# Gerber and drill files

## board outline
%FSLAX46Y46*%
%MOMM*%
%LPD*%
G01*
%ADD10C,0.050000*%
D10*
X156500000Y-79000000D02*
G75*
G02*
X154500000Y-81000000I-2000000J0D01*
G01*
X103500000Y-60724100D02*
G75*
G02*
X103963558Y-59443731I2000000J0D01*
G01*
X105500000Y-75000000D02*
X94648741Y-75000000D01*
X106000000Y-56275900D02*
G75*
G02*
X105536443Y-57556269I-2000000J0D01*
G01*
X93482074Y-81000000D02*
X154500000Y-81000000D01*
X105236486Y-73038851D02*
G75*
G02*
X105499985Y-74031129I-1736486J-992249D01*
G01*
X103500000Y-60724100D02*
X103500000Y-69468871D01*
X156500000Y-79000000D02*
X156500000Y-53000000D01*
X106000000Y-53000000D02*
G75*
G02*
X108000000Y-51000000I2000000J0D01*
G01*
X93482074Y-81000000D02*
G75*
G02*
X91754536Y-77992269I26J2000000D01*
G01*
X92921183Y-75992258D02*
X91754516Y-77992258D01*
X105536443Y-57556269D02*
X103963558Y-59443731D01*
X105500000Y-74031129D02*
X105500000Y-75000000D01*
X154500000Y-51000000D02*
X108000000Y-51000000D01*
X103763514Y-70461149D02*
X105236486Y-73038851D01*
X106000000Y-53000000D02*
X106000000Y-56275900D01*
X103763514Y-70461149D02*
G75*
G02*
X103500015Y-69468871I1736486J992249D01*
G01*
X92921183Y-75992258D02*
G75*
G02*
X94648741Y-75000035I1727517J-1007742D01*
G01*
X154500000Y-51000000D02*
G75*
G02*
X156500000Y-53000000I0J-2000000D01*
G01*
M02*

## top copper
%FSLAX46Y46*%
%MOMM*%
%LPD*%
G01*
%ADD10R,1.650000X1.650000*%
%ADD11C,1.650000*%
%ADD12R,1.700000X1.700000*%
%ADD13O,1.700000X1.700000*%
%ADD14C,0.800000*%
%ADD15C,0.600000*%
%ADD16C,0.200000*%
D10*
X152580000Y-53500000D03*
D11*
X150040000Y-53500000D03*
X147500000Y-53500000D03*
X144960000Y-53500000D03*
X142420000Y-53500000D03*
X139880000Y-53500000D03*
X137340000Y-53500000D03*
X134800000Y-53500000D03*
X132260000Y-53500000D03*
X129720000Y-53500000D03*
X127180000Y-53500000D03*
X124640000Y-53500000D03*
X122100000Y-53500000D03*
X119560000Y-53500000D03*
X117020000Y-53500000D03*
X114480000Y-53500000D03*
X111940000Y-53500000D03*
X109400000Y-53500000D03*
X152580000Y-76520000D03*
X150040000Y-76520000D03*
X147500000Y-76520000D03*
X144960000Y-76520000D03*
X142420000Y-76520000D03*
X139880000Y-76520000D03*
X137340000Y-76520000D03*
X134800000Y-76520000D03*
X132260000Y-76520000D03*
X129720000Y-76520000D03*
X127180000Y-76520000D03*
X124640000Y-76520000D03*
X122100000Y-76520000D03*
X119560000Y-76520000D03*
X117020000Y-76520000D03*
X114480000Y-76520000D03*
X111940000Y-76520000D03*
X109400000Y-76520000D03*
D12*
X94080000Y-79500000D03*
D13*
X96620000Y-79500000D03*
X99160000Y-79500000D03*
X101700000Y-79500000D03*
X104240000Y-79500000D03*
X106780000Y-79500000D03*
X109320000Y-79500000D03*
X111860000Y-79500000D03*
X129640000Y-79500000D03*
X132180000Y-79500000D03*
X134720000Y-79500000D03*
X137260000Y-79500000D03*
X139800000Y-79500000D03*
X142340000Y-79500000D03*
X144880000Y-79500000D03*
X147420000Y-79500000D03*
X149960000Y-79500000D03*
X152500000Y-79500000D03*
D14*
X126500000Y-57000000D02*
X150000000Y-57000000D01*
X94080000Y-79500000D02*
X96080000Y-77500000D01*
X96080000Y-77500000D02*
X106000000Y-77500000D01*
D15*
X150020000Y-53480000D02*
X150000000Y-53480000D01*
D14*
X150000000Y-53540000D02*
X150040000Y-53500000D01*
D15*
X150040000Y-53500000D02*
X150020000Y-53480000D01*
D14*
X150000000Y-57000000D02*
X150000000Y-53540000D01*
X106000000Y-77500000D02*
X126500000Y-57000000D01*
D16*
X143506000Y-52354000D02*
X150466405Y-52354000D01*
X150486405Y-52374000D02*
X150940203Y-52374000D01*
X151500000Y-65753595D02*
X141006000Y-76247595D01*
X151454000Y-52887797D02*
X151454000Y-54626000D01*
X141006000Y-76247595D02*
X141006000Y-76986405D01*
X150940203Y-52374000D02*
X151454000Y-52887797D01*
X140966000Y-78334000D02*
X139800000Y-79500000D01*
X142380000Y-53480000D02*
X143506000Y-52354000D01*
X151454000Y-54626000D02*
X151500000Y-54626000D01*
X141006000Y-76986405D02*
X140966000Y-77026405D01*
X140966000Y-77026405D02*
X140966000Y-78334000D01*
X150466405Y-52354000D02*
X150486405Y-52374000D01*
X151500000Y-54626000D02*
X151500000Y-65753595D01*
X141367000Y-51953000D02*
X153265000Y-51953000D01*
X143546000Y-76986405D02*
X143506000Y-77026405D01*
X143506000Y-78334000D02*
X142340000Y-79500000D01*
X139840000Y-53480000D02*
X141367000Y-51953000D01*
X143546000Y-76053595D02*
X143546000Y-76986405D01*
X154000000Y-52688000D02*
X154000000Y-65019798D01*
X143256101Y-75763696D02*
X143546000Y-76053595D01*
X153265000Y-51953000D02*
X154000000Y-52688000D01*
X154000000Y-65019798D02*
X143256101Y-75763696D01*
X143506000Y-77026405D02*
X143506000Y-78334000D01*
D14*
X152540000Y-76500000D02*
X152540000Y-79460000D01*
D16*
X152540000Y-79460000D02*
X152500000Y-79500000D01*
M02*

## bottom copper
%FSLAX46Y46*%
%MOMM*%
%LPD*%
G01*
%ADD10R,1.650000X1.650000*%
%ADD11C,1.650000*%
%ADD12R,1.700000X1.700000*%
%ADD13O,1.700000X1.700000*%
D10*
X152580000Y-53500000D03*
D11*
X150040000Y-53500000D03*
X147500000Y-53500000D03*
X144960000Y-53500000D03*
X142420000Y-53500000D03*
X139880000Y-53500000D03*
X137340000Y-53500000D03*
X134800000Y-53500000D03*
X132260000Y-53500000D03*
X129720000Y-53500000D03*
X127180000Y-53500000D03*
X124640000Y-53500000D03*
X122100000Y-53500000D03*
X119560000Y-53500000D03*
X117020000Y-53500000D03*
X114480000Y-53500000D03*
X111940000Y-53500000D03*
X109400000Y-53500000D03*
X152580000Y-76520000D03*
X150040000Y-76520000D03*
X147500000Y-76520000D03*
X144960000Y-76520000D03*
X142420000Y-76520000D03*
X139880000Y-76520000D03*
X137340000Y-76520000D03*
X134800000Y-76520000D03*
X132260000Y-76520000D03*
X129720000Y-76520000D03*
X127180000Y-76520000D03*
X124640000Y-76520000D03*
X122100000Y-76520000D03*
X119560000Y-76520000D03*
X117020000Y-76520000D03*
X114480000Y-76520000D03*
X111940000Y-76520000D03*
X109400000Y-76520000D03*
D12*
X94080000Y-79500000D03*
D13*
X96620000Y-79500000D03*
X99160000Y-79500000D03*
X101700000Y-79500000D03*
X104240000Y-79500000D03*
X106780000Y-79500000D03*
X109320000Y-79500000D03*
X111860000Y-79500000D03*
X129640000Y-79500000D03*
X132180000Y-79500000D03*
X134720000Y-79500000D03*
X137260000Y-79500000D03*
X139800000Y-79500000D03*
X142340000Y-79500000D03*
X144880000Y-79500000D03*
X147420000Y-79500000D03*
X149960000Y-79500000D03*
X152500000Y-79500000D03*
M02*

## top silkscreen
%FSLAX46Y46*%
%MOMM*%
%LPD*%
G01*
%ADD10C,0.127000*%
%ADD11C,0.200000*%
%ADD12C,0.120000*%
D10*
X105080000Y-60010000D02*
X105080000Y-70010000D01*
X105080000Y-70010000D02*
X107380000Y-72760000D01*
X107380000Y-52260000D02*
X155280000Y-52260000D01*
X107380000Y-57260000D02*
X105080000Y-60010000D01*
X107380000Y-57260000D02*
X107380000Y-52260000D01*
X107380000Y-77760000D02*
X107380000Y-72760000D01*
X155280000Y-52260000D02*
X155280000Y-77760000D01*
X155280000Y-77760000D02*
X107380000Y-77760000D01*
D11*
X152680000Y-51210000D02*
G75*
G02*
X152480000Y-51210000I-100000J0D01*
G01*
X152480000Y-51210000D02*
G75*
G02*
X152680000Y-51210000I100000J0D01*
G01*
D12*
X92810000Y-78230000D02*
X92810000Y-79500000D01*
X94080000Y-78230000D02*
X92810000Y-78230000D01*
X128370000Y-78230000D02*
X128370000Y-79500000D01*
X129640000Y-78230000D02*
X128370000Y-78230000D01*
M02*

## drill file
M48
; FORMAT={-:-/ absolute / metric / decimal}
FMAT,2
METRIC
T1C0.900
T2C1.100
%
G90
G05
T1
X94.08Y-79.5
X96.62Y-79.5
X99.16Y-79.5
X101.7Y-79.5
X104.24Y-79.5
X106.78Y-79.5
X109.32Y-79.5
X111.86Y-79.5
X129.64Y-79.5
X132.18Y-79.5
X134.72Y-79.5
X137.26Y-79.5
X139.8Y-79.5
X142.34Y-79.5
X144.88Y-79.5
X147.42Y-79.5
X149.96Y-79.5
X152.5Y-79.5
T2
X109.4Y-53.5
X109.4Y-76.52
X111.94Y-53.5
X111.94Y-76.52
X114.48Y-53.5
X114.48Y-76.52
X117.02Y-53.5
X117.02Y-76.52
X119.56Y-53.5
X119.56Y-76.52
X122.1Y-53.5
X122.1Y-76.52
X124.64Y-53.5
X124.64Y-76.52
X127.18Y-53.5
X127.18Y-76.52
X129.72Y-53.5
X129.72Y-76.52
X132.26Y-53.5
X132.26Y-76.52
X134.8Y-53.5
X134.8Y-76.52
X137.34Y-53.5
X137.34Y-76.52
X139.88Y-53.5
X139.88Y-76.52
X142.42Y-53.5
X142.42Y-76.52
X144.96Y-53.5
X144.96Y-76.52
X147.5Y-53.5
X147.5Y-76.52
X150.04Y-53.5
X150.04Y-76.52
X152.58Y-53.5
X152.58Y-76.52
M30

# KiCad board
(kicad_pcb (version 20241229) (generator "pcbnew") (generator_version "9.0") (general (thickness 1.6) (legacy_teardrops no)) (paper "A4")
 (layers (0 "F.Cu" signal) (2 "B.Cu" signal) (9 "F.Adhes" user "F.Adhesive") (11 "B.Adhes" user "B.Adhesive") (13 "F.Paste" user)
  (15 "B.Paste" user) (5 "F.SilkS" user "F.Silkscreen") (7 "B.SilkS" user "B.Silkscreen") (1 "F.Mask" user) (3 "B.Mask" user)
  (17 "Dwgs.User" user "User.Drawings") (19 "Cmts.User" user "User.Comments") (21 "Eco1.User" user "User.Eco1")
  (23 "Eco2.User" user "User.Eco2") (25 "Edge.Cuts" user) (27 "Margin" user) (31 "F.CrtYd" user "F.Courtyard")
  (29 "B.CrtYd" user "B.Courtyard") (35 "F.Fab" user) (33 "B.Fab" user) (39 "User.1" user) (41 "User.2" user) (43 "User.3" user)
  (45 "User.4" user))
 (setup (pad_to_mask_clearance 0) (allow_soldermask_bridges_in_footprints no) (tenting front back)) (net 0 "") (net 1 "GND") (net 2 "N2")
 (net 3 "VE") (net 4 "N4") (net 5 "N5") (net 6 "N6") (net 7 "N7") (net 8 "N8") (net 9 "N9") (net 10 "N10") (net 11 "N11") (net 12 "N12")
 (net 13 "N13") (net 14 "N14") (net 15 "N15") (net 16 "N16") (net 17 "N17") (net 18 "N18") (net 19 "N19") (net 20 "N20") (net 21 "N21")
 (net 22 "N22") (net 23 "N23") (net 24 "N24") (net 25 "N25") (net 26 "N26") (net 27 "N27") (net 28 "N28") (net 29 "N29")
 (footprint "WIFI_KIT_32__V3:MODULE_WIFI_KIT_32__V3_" (layer "F.Cu") (at 130.18 65.01 -90)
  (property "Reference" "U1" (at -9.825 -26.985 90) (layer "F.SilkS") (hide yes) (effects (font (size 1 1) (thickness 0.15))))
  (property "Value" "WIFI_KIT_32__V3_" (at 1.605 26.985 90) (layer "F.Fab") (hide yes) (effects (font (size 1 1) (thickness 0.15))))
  (fp_line (start -5 25.1) (end 5 25.1) (stroke (width 0.127) (type solid)) (layer "F.SilkS"))
  (fp_line (start 5 25.1) (end 7.75 22.8) (stroke (width 0.127) (type solid)) (layer "F.SilkS"))
  (fp_line (start -12.75 22.8) (end -12.75 -25.1) (stroke (width 0.127) (type solid)) (layer "F.SilkS"))
  (fp_line (start -7.75 22.8) (end -5 25.1) (stroke (width 0.127) (type solid)) (layer "F.SilkS"))
  (fp_line (start -7.75 22.8) (end -12.75 22.8) (stroke (width 0.127) (type solid)) (layer "F.SilkS"))
  (fp_line (start 12.75 22.8) (end 7.75 22.8) (stroke (width 0.127) (type solid)) (layer "F.SilkS"))
  (fp_line (start -12.75 -25.1) (end 12.75 -25.1) (stroke (width 0.127) (type solid)) (layer "F.SilkS"))
  (fp_line (start 12.75 -25.1) (end 12.75 22.8) (stroke (width 0.127) (type solid)) (layer "F.SilkS"))
  (fp_circle (center -13.8 -22.4) (end -13.7 -22.4) (stroke (width 0.2) (type solid)) (fill no) (layer "F.SilkS"))
  (pad "J2_1" thru_hole rect (at -11.51 -22.4 270) (size 1.65 1.65) (drill 1.1) (layers "*.Cu" "*.Mask") (remove_unused_layers no)
   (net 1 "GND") (solder_mask_margin 0.102))
  (pad "J2_2" thru_hole circle (at -11.51 -19.86 270) (size 1.65 1.65) (drill 1.1) (layers "*.Cu" "*.Mask") (remove_unused_layers no)
   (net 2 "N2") (solder_mask_margin 0.102))
  (pad "J2_3" thru_hole circle (at -11.51 -17.32 270) (size 1.65 1.65) (drill 1.1) (layers "*.Cu" "*.Mask") (remove_unused_layers no)
   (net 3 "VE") (solder_mask_margin 0.102))
  (pad "J2_4" thru_hole circle (at -11.51 -14.78 270) (size 1.65 1.65) (drill 1.1) (layers "*.Cu" "*.Mask") (remove_unused_layers no)
   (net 3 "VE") (solder_mask_margin 0.102))
  (pad "J2_5" thru_hole circle (at -11.51 -12.24 270) (size 1.65 1.65) (drill 1.1) (layers "*.Cu" "*.Mask") (remove_unused_layers no)
   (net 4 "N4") (solder_mask_margin 0.102))
  (pad "J2_6" thru_hole circle (at -11.51 -9.7 270) (size 1.65 1.65) (drill 1.1) (layers "*.Cu" "*.Mask") (remove_unused_layers no)
   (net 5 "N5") (solder_mask_margin 0.102))
  (pad "J2_7" thru_hole circle (at -11.51 -7.16 270) (size 1.65 1.65) (drill 1.1) (layers "*.Cu" "*.Mask") (remove_unused_layers no)
   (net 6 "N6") (solder_mask_margin 0.102))
  (pad "J2_8" thru_hole circle (at -11.51 -4.62 270) (size 1.65 1.65) (drill 1.1) (layers "*.Cu" "*.Mask") (remove_unused_layers no)
   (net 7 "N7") (solder_mask_margin 0.102))
  (pad "J2_9" thru_hole circle (at -11.51 -2.08 270) (size 1.65 1.65) (drill 1.1) (layers "*.Cu" "*.Mask") (remove_unused_layers no)
   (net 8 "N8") (solder_mask_margin 0.102))
  (pad "J2_10" thru_hole circle (at -11.51 0.46 270) (size 1.65 1.65) (drill 1.1) (layers "*.Cu" "*.Mask") (remove_unused_layers no)
   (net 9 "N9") (solder_mask_margin 0.102))
  (pad "J2_11" thru_hole circle (at -11.51 3 270) (size 1.65 1.65) (drill 1.1) (layers "*.Cu" "*.Mask") (remove_unused_layers no)
   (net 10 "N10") (solder_mask_margin 0.102))
  (pad "J2_12" thru_hole circle (at -11.51 5.54 270) (size 1.65 1.65) (drill 1.1) (layers "*.Cu" "*.Mask") (remove_unused_layers no)
   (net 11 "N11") (solder_mask_margin 0.102))
  (pad "J2_13" thru_hole circle (at -11.51 8.08 270) (size 1.65 1.65) (drill 1.1) (layers "*.Cu" "*.Mask") (remove_unused_layers no)
   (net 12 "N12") (solder_mask_margin 0.102))
  (pad "J2_14" thru_hole circle (at -11.51 10.62 270) (size 1.65 1.65) (drill 1.1) (layers "*.Cu" "*.Mask") (remove_unused_layers no)
   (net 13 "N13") (solder_mask_margin 0.102))
  (pad "J2_15" thru_hole circle (at -11.51 13.16 270) (size 1.65 1.65) (drill 1.1) (layers "*.Cu" "*.Mask") (remove_unused_layers no)
   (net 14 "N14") (solder_mask_margin 0.102))
  (pad "J2_16" thru_hole circle (at -11.51 15.7 270) (size 1.65 1.65) (drill 1.1) (layers "*.Cu" "*.Mask") (remove_unused_layers no)
   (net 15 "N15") (solder_mask_margin 0.102))
  (pad "J2_17" thru_hole circle (at -11.51 18.24 270) (size 1.65 1.65) (drill 1.1) (layers "*.Cu" "*.Mask") (remove_unused_layers no)
   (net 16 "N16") (solder_mask_margin 0.102))
  (pad "J2_18" thru_hole circle (at -11.51 20.78 270) (size 1.65 1.65) (drill 1.1) (layers "*.Cu" "*.Mask") (remove_unused_layers no)
   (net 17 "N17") (solder_mask_margin 0.102))
  (pad "J3_1" thru_hole circle (at 11.51 -22.4 270) (size 1.65 1.65) (drill 1.1) (layers "*.Cu" "*.Mask") (remove_unused_layers no)
   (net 1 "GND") (solder_mask_margin 0.102))
  (pad "J3_2" thru_hole circle (at 11.51 -19.86 270) (size 1.65 1.65) (drill 1.1) (layers "*.Cu" "*.Mask") (remove_unused_layers no)
   (solder_mask_margin 0.102))
  (pad "J3_3" thru_hole circle (at 11.51 -17.32 270) (size 1.65 1.65) (drill 1.1) (layers "*.Cu" "*.Mask") (remove_unused_layers no)
   (solder_mask_margin 0.102))
  (pad "J3_4" thru_hole circle (at 11.51 -14.78 270) (size 1.65 1.65) (drill 1.1) (layers "*.Cu" "*.Mask") (remove_unused_layers no)
   (solder_mask_margin 0.102))
  (pad "J3_5" thru_hole circle (at 11.51 -12.24 270) (size 1.65 1.65) (drill 1.1) (layers "*.Cu" "*.Mask") (remove_unused_layers no)
   (solder_mask_margin 0.102))
  (pad "J3_6" thru_hole circle (at 11.51 -9.7 270) (size 1.65 1.65) (drill 1.1) (layers "*.Cu" "*.Mask") (remove_unused_layers no)
   (solder_mask_margin 0.102))
  (pad "J3_7" thru_hole circle (at 11.51 -7.16 270) (size 1.65 1.65) (drill 1.1) (layers "*.Cu" "*.Mask") (remove_unused_layers no)
   (solder_mask_margin 0.102))
  (pad "J3_8" thru_hole circle (at 11.51 -4.62 270) (size 1.65 1.65) (drill 1.1) (layers "*.Cu" "*.Mask") (remove_unused_layers no)
   (solder_mask_margin 0.102))
  (pad "J3_9" thru_hole circle (at 11.51 -2.08 270) (size 1.65 1.65) (drill 1.1) (layers "*.Cu" "*.Mask") (remove_unused_layers no)
   (solder_mask_margin 0.102))
  (pad "J3_10" thru_hole circle (at 11.51 0.46 270) (size 1.65 1.65) (drill 1.1) (layers "*.Cu" "*.Mask") (remove_unused_layers no)
   (solder_mask_margin 0.102))
  (pad "J3_11" thru_hole circle (at 11.51 3 270) (size 1.65 1.65) (drill 1.1) (layers "*.Cu" "*.Mask") (remove_unused_layers no)
   (solder_mask_margin 0.102))
  (pad "J3_12" thru_hole circle (at 11.51 5.54 270) (size 1.65 1.65) (drill 1.1) (layers "*.Cu" "*.Mask") (remove_unused_layers no)
   (solder_mask_margin 0.102))
  (pad "J3_13" thru_hole circle (at 11.51 8.08 270) (size 1.65 1.65) (drill 1.1) (layers "*.Cu" "*.Mask") (remove_unused_layers no)
   (solder_mask_margin 0.102))
  (pad "J3_14" thru_hole circle (at 11.51 10.62 270) (size 1.65 1.65) (drill 1.1) (layers "*.Cu" "*.Mask") (remove_unused_layers no)
   (solder_mask_margin 0.102))
  (pad "J3_15" thru_hole circle (at 11.51 13.16 270) (size 1.65 1.65) (drill 1.1) (layers "*.Cu" "*.Mask") (remove_unused_layers no)
   (solder_mask_margin 0.102))
  (pad "J3_16" thru_hole circle (at 11.51 15.7 270) (size 1.65 1.65) (drill 1.1) (layers "*.Cu" "*.Mask") (remove_unused_layers no)
   (solder_mask_margin 0.102))
  (pad "J3_17" thru_hole circle (at 11.51 18.24 270) (size 1.65 1.65) (drill 1.1) (layers "*.Cu" "*.Mask") (remove_unused_layers no)
   (solder_mask_margin 0.102))
  (pad "J3_18" thru_hole circle (at 11.51 20.78 270) (size 1.65 1.65) (drill 1.1) (layers "*.Cu" "*.Mask") (remove_unused_layers no)
   (solder_mask_margin 0.102)))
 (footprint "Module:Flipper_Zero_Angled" (layer "F.Cu") (at 94.08 79.5)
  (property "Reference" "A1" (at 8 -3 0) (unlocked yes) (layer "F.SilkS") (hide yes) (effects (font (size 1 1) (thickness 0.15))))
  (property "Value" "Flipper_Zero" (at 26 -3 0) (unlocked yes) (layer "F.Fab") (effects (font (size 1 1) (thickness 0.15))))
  (fp_line (start -1.27 -1.27) (end -1.27 0) (stroke (width 0.12) (type solid)) (layer "F.SilkS"))
  (fp_line (start 0 -1.27) (end -1.27 -1.27) (stroke (width 0.12) (type solid)) (layer "F.SilkS"))
  (fp_line (start 34.29 -1.27) (end 34.29 0) (stroke (width 0.12) (type solid)) (layer "F.SilkS"))
  (fp_line (start 35.56 -1.27) (end 34.29 -1.27) (stroke (width 0.12) (type solid)) (layer "F.SilkS"))
  (pad "1" thru_hole rect (at 0 0 90) (size 1.7 1.7) (drill 0.9) (layers "*.Cu" "*.Mask") (remove_unused_layers no) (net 2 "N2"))
  (pad "2" thru_hole oval (at 2.54 0 90) (size 1.7 1.7) (drill 0.9) (layers "*.Cu" "*.Mask") (remove_unused_layers no) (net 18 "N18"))
  (pad "3" thru_hole oval (at 5.08 0 90) (size 1.7 1.7) (drill 0.9) (layers "*.Cu" "*.Mask") (remove_unused_layers no) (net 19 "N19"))
  (pad "4" thru_hole oval (at 7.62 0 90) (size 1.7 1.7) (drill 0.9) (layers "*.Cu" "*.Mask") (remove_unused_layers no) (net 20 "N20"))
  (pad "5" thru_hole oval (at 10.16 0 90) (size 1.7 1.7) (drill 0.9) (layers "*.Cu" "*.Mask") (remove_unused_layers no) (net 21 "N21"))
  (pad "6" thru_hole oval (at 12.7 0 90) (size 1.7 1.7) (drill 0.9) (layers "*.Cu" "*.Mask") (remove_unused_layers no) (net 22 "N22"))
  (pad "7" thru_hole oval (at 15.24 0 90) (size 1.7 1.7) (drill 0.9) (layers "*.Cu" "*.Mask") (remove_unused_layers no) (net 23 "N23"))
  (pad "8" thru_hole oval (at 17.78 0 90) (size 1.7 1.7) (drill 0.9) (layers "*.Cu" "*.Mask") (remove_unused_layers no) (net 1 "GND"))
  (pad "9" thru_hole oval (at 35.56 0 90) (size 1.7 1.7) (drill 0.9) (layers "*.Cu" "*.Mask") (remove_unused_layers no) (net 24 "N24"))
  (pad "10" thru_hole oval (at 38.1 0 90) (size 1.7 1.7) (drill 0.9) (layers "*.Cu" "*.Mask") (remove_unused_layers no) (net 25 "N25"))
  (pad "11" thru_hole oval (at 40.64 0 90) (size 1.7 1.7) (drill 0.9) (layers "*.Cu" "*.Mask") (remove_unused_layers no) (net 1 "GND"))
  (pad "12" thru_hole oval (at 43.18 0 90) (size 1.7 1.7) (drill 0.9) (layers "*.Cu" "*.Mask") (remove_unused_layers no) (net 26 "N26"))
  (pad "13" thru_hole oval (at 45.72 0 90) (size 1.7 1.7) (drill 0.9) (layers "*.Cu" "*.Mask") (remove_unused_layers no) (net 4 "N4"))
  (pad "14" thru_hole oval (at 48.26 0 90) (size 1.7 1.7) (drill 0.9) (layers "*.Cu" "*.Mask") (remove_unused_layers no) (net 5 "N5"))
  (pad "15" thru_hole oval (at 50.8 0 90) (size 1.7 1.7) (drill 0.9) (layers "*.Cu" "*.Mask") (remove_unused_layers no) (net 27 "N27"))
  (pad "16" thru_hole oval (at 53.34 0 90) (size 1.7 1.7) (drill 0.9) (layers "*.Cu" "*.Mask") (remove_unused_layers no) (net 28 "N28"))
  (pad "17" thru_hole oval (at 55.88 0 90) (size 1.7 1.7) (drill 0.9) (layers "*.Cu" "*.Mask") (remove_unused_layers no) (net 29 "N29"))
  (pad "18" thru_hole oval (at 58.42 0 90) (size 1.7 1.7) (drill 0.9) (layers "*.Cu" "*.Mask") (remove_unused_layers no) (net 1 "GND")))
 (gr_arc (start 156.5 79) (mid 155.914214 80.414214) (end 154.5 81) (stroke (width 0.05) (type default)) (layer "Edge.Cuts"))
 (gr_arc (start 103.5 60.7241) (mid 103.619457 60.043249) (end 103.963558 59.443731) (stroke (width 0.05) (type default))
  (layer "Edge.Cuts"))
 (gr_line (start 105.5 75) (end 94.648741 75) (stroke (width 0.05) (type default)) (layer "Edge.Cuts"))
 (gr_arc (start 106 56.2759) (mid 105.880543 56.95675) (end 105.536443 57.556269) (stroke (width 0.05) (type default)) (layer "Edge.Cuts"))
 (gr_line (start 93.482074 81) (end 154.5 81) (stroke (width 0.05) (type default)) (layer "Edge.Cuts"))
 (gr_arc (start 105.236486 73.038851) (mid 105.432999 73.517793) (end 105.5 74.031129) (stroke (width 0.05) (type default))
  (layer "Edge.Cuts"))
 (gr_line (start 103.5 60.7241) (end 103.5 69.468871) (stroke (width 0.05) (type default)) (layer "Edge.Cuts"))
 (gr_line (start 156.5 79) (end 156.5 53) (stroke (width 0.05) (type default)) (layer "Edge.Cuts"))
 (gr_arc (start 106 53) (mid 106.585786 51.585786) (end 108 51) (stroke (width 0.05) (type default)) (layer "Edge.Cuts"))
 (gr_arc (start 93.482074 81) (mid 91.747813 79.996116) (end 91.754516 77.992258) (stroke (width 0.05) (type default)) (layer "Edge.Cuts"))
 (gr_line (start 92.921183 75.992258) (end 91.754516 77.992258) (stroke (width 0.05) (type default)) (layer "Edge.Cuts"))
 (gr_line (start 105.536443 57.556269) (end 103.963558 59.443731) (stroke (width 0.05) (type default)) (layer "Edge.Cuts"))
 (gr_line (start 105.5 74.031129) (end 105.5 75) (stroke (width 0.05) (type default)) (layer "Edge.Cuts"))
 (gr_line (start 154.5 51) (end 108 51) (stroke (width 0.05) (type default)) (layer "Edge.Cuts"))
 (gr_line (start 103.763514 70.461149) (end 105.236486 73.038851) (stroke (width 0.05) (type default)) (layer "Edge.Cuts"))
 (gr_line (start 106 53) (end 106 56.2759) (stroke (width 0.05) (type default)) (layer "Edge.Cuts"))
 (gr_arc (start 103.763514 70.461149) (mid 103.567001 69.982207) (end 103.5 69.468871) (stroke (width 0.05) (type default))
  (layer "Edge.Cuts"))
 (gr_arc (start 92.921183 75.992258) (mid 93.652619 75.265716) (end 94.648741 75) (stroke (width 0.05) (type default)) (layer "Edge.Cuts"))
 (gr_arc (start 154.5 51) (mid 155.914214 51.585786) (end 156.5 53) (stroke (width 0.05) (type default)) (layer "Edge.Cuts"))
 (segment (start 126.5 57) (end 150 57) (width 0.8) (layer "F.Cu") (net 2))
 (segment (start 94.08 79.5) (end 96.08 77.5) (width 0.8) (layer "F.Cu") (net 2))
 (segment (start 96.08 77.5) (end 106 77.5) (width 0.8) (layer "F.Cu") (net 2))
 (segment (start 150.02 53.48) (end 150 53.48) (width 0.6) (layer "F.Cu") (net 2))
 (segment (start 150 53.54) (end 150.04 53.5) (width 0.8) (layer "F.Cu") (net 2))
 (segment (start 150.04 53.5) (end 150.02 53.48) (width 0.6) (layer "F.Cu") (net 2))
 (segment (start 150 57) (end 150 53.54) (width 0.8) (layer "F.Cu") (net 2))
 (segment (start 106 77.5) (end 126.5 57) (width 0.8) (layer "F.Cu") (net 2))
 (segment (start 143.506 52.354) (end 150.466405 52.354) (width 0.2) (layer "F.Cu") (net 4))
 (segment (start 150.486405 52.374) (end 150.940203 52.374) (width 0.2) (layer "F.Cu") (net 4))
 (segment (start 151.5 65.753595) (end 141.006 76.247595) (width 0.2) (layer "F.Cu") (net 4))
 (segment (start 151.454 52.887797) (end 151.454 54.626) (width 0.2) (layer "F.Cu") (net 4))
 (segment (start 141.006 76.247595) (end 141.006 76.986405) (width 0.2) (layer "F.Cu") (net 4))
 (segment (start 150.940203 52.374) (end 151.454 52.887797) (width 0.2) (layer "F.Cu") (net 4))
 (segment (start 140.966 78.334) (end 139.8 79.5) (width 0.2) (layer "F.Cu") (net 4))
 (segment (start 142.38 53.48) (end 143.506 52.354) (width 0.2) (layer "F.Cu") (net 4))
 (segment (start 151.454 54.626) (end 151.5 54.626) (width 0.2) (layer "F.Cu") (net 4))
 (segment (start 141.006 76.986405) (end 140.966 77.026405) (width 0.2) (layer "F.Cu") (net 4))
 (segment (start 140.966 77.026405) (end 140.966 78.334) (width 0.2) (layer "F.Cu") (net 4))
 (segment (start 150.466405 52.354) (end 150.486405 52.374) (width 0.2) (layer "F.Cu") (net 4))
 (segment (start 151.5 54.626) (end 151.5 65.753595) (width 0.2) (layer "F.Cu") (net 4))
 (segment (start 141.367 51.953) (end 153.265 51.953) (width 0.2) (layer "F.Cu") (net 5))
 (segment (start 143.546 76.986405) (end 143.506 77.026405) (width 0.2) (layer "F.Cu") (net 5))
 (segment (start 143.506 78.334) (end 142.34 79.5) (width 0.2) (layer "F.Cu") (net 5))
 (segment (start 139.84 53.48) (end 141.367 51.953) (width 0.2) (layer "F.Cu") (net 5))
 (segment (start 143.546 76.053595) (end 143.546 76.986405) (width 0.2) (layer "F.Cu") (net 5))
 (segment (start 154 52.688) (end 154 65.019798) (width 0.2) (layer "F.Cu") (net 5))
 (segment (start 143.256101 75.763696) (end 143.546 76.053595) (width 0.2) (layer "F.Cu") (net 5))
 (segment (start 153.265 51.953) (end 154 52.688) (width 0.2) (layer "F.Cu") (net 5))
 (segment (start 154 65.019798) (end 143.256101 75.763696) (width 0.2) (layer "F.Cu") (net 5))
 (segment (start 143.506 77.026405) (end 143.506 78.334) (width 0.2) (layer "F.Cu") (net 5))
 (segment (start 152.54 76.5) (end 152.54 79.46) (width 0.8) (layer "F.Cu") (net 1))
 (segment (start 152.54 79.46) (end 152.5 79.5) (width 0.2) (layer "F.Cu") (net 1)))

